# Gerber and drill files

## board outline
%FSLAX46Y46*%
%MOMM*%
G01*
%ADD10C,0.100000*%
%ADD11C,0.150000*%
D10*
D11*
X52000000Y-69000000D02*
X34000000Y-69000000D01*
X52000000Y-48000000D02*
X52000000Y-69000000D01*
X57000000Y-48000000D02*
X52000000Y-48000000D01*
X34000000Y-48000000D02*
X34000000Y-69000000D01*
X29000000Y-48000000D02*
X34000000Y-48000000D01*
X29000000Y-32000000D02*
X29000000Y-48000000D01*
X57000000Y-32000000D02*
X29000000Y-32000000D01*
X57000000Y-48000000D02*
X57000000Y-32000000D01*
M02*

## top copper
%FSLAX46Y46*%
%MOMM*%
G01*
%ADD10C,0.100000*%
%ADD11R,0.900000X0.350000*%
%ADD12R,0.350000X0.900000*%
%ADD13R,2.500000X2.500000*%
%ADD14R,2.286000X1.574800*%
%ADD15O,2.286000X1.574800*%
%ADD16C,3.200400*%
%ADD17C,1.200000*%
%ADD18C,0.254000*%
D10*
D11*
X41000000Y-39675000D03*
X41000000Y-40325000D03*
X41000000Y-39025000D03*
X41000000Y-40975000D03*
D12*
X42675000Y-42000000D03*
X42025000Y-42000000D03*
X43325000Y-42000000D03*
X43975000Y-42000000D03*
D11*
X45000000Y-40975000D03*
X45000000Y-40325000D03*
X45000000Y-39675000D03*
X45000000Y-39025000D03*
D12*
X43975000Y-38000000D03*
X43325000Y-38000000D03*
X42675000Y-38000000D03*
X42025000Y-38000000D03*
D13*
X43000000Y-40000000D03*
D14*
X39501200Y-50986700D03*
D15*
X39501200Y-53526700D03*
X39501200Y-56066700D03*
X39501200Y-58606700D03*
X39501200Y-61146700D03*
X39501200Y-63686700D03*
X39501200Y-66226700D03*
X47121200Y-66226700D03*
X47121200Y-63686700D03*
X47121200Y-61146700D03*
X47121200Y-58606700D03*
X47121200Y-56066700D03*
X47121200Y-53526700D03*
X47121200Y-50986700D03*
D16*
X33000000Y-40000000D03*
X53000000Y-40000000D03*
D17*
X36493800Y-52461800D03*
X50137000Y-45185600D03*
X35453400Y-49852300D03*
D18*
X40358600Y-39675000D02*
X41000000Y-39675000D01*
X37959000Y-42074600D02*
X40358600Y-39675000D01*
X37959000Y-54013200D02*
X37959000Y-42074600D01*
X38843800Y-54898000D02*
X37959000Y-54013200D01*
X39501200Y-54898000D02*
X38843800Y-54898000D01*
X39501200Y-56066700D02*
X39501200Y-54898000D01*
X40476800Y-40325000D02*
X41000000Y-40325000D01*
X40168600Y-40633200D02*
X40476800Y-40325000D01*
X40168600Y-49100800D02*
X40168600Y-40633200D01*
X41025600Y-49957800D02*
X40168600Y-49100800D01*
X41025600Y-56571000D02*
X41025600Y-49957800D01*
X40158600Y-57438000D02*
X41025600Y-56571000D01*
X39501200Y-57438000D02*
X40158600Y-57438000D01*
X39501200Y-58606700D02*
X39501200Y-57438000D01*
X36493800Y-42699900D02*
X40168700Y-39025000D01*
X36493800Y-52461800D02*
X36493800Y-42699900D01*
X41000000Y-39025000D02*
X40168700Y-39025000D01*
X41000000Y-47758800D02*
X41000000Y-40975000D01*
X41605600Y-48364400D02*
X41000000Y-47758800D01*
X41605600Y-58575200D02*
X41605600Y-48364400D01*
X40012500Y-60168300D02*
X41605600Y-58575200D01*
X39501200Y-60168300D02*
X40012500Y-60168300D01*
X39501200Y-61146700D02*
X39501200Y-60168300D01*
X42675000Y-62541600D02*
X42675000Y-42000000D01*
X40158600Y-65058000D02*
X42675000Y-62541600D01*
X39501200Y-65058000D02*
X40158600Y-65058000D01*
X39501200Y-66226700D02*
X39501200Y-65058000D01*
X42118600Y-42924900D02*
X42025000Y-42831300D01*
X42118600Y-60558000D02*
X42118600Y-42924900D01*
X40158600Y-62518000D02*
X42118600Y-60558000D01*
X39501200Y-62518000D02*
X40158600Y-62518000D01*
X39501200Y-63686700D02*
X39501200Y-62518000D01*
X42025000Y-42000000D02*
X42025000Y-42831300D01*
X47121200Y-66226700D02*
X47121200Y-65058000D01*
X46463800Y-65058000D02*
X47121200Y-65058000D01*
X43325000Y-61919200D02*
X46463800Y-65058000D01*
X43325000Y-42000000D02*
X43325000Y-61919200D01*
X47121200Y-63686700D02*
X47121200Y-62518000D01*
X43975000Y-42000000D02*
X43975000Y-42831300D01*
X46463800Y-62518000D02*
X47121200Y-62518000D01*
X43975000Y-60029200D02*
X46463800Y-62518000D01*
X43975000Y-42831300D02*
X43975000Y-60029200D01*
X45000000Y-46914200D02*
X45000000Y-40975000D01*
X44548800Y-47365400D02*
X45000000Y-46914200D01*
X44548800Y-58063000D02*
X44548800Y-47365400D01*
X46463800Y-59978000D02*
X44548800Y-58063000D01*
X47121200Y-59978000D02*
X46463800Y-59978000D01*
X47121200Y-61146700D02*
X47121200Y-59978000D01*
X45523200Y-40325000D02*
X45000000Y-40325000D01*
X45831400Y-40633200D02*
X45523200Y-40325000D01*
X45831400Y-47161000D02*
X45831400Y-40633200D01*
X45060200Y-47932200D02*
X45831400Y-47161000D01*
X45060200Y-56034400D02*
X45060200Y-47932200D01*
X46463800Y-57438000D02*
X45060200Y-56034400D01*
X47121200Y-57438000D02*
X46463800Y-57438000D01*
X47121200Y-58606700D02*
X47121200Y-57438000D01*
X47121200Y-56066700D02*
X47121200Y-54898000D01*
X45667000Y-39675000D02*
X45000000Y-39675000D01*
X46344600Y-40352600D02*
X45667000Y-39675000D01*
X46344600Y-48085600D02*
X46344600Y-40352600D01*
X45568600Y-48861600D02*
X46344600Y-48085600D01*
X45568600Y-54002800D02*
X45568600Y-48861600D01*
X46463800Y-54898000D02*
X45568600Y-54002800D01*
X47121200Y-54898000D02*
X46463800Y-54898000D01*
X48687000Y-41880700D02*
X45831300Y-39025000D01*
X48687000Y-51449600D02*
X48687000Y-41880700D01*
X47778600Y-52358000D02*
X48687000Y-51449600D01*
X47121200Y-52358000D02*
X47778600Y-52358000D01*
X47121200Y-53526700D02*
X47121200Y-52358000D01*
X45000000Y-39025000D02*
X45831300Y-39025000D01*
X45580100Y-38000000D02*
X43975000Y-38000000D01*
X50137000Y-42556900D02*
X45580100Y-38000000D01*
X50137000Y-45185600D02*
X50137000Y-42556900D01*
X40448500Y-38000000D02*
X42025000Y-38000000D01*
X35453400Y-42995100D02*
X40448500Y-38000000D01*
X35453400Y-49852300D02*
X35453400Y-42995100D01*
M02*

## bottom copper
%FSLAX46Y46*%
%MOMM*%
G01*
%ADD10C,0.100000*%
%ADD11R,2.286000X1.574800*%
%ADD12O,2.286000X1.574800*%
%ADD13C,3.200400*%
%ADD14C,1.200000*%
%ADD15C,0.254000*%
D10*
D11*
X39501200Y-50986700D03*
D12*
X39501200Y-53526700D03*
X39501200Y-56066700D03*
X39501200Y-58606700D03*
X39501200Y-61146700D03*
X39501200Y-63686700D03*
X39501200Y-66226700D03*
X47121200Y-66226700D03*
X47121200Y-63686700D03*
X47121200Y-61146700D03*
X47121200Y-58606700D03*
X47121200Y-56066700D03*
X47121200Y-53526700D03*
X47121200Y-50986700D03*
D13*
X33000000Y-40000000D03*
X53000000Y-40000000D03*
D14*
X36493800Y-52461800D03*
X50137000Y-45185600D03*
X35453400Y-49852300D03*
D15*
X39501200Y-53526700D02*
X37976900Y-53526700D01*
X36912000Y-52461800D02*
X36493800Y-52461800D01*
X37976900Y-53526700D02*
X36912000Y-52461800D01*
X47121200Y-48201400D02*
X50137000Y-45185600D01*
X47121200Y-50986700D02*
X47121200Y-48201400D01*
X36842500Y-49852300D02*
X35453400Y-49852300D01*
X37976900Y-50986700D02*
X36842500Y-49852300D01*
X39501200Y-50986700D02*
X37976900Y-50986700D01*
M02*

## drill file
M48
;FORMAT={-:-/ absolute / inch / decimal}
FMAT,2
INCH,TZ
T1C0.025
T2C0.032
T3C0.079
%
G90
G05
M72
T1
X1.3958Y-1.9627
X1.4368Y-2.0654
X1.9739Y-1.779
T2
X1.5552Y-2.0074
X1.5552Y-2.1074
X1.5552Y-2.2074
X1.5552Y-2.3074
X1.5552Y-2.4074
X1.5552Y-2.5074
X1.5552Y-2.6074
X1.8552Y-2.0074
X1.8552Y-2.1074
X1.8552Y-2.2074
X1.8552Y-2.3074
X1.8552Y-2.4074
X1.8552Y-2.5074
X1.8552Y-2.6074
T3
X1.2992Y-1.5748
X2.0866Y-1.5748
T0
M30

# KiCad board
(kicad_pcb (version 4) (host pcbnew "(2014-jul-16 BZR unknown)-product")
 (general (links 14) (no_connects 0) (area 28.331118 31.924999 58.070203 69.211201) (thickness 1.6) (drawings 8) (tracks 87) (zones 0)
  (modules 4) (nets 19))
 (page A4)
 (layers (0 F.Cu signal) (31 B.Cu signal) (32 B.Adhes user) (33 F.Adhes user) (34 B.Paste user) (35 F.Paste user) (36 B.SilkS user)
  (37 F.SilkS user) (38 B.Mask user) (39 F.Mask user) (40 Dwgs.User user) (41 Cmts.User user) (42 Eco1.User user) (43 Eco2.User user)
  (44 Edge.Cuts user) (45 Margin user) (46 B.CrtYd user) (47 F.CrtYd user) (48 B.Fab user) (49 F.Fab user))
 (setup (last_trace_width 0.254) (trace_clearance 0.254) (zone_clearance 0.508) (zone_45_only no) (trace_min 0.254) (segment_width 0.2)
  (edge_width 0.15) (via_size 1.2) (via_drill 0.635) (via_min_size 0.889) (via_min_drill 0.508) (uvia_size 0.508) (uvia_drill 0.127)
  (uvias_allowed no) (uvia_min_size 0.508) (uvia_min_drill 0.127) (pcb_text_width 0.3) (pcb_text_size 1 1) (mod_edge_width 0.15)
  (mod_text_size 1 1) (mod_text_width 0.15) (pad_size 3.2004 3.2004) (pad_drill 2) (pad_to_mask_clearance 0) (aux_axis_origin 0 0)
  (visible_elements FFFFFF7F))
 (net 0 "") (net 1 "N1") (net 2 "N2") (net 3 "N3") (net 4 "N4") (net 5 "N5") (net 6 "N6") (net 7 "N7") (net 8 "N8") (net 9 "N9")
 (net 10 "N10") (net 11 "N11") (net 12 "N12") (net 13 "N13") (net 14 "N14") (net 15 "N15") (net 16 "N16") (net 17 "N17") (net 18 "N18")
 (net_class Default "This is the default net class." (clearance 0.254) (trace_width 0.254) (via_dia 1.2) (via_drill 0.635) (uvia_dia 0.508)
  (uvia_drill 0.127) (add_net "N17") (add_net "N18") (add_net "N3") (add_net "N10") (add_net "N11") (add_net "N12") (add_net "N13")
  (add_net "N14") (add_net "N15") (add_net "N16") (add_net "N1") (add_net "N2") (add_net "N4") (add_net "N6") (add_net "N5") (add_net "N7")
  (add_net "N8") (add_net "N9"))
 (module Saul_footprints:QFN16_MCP (layer F.Cu) (at 43 40)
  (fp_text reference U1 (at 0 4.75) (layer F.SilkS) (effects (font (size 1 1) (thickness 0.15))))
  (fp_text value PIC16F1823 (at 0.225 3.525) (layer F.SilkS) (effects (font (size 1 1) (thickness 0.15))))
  (pad 2 smd rect (at -2 -0.325) (size 0.9 0.35) (layers F.Cu F.Paste F.Mask) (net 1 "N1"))
  (pad 3 smd rect (at -2 0.325) (size 0.9 0.35) (layers F.Cu F.Paste F.Mask) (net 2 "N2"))
  (pad 1 smd rect (at -2 -0.975) (size 0.9 0.35) (layers F.Cu F.Paste F.Mask) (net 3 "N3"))
  (pad 4 smd rect (at -2 0.975) (size 0.9 0.35) (layers F.Cu F.Paste F.Mask) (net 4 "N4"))
  (pad 6 smd rect (at -0.325 2 90) (size 0.9 0.35) (layers F.Cu F.Paste F.Mask) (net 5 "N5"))
  (pad 5 smd rect (at -0.975 2 90) (size 0.9 0.35) (layers F.Cu F.Paste F.Mask) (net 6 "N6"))
  (pad 7 smd rect (at 0.325 2 90) (size 0.9 0.35) (layers F.Cu F.Paste F.Mask) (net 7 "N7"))
  (pad 8 smd rect (at 0.975 2 90) (size 0.9 0.35) (layers F.Cu F.Paste F.Mask) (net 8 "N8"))
  (pad 9 smd rect (at 2 0.975) (size 0.9 0.35) (layers F.Cu F.Paste F.Mask) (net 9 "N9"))
  (pad 10 smd rect (at 2 0.325) (size 0.9 0.35) (layers F.Cu F.Paste F.Mask) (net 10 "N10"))
  (pad 11 smd rect (at 2 -0.325) (size 0.9 0.35) (layers F.Cu F.Paste F.Mask) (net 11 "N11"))
  (pad 12 smd rect (at 2 -0.975) (size 0.9 0.35) (layers F.Cu F.Paste F.Mask) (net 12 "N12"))
  (pad 13 smd rect (at 0.975 -2 90) (size 0.9 0.35) (layers F.Cu F.Paste F.Mask) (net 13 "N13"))
  (pad 14 smd rect (at 0.325 -2 90) (size 0.9 0.35) (layers F.Cu F.Paste F.Mask) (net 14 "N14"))
  (pad 15 smd rect (at -0.325 -2 90) (size 0.9 0.35) (layers F.Cu F.Paste F.Mask) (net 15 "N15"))
  (pad 16 smd rect (at -0.975 -2 90) (size 0.9 0.35) (layers F.Cu F.Paste F.Mask) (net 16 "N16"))
  (pad "" smd rect (at 0 0 90) (size 2.5 2.5) (layers F.Cu F.Paste F.Mask)))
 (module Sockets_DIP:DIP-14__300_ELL (layer F.Cu) (at 43.3112 58.6067 270)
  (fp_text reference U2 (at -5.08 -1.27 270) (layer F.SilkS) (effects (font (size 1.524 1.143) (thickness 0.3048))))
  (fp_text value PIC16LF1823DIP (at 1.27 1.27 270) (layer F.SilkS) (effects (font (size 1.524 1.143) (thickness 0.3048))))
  (pad 1 thru_hole rect (at -7.62 3.81 270) (size 1.5748 2.286) (drill 0.8128) (layers *.Cu *.Mask F.SilkS) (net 16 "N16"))
  (pad 2 thru_hole oval (at -5.08 3.81 270) (size 1.5748 2.286) (drill 0.8128) (layers *.Cu *.Mask F.SilkS) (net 3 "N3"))
  (pad 3 thru_hole oval (at -2.54 3.81 270) (size 1.5748 2.286) (drill 0.8128) (layers *.Cu *.Mask F.SilkS) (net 1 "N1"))
  (pad 4 thru_hole oval (at 0 3.81 270) (size 1.5748 2.286) (drill 0.8128) (layers *.Cu *.Mask F.SilkS) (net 2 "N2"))
  (pad 5 thru_hole oval (at 2.54 3.81 270) (size 1.5748 2.286) (drill 0.8128) (layers *.Cu *.Mask F.SilkS) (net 4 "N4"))
  (pad 6 thru_hole oval (at 5.08 3.81 270) (size 1.5748 2.286) (drill 0.8128) (layers *.Cu *.Mask F.SilkS) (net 6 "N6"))
  (pad 7 thru_hole oval (at 7.62 3.81 270) (size 1.5748 2.286) (drill 0.8128) (layers *.Cu *.Mask F.SilkS) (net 5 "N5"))
  (pad 8 thru_hole oval (at 7.62 -3.81 270) (size 1.5748 2.286) (drill 0.8128) (layers *.Cu *.Mask F.SilkS) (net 7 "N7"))
  (pad 9 thru_hole oval (at 5.08 -3.81 270) (size 1.5748 2.286) (drill 0.8128) (layers *.Cu *.Mask F.SilkS) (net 8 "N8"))
  (pad 10 thru_hole oval (at 2.54 -3.81 270) (size 1.5748 2.286) (drill 0.8128) (layers *.Cu *.Mask F.SilkS) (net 9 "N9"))
  (pad 11 thru_hole oval (at 0 -3.81 270) (size 1.5748 2.286) (drill 0.8128) (layers *.Cu *.Mask F.SilkS) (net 10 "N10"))
  (pad 12 thru_hole oval (at -2.54 -3.81 270) (size 1.5748 2.286) (drill 0.8128) (layers *.Cu *.Mask F.SilkS) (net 11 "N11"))
  (pad 13 thru_hole oval (at -5.08 -3.81 270) (size 1.5748 2.286) (drill 0.8128) (layers *.Cu *.Mask F.SilkS) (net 12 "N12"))
  (pad 14 thru_hole oval (at -7.62 -3.81 270) (size 1.5748 2.286) (drill 0.8128) (layers *.Cu *.Mask F.SilkS) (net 13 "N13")))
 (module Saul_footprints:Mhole (layer F.Cu) (at 33 40)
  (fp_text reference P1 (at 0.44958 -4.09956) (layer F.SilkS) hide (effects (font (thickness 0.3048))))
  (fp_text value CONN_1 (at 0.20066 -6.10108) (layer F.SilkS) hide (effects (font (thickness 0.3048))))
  (pad 1 thru_hole circle (at 0 0) (size 3.2004 3.2004) (drill 2) (layers *.Cu *.Mask F.SilkS) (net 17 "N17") (clearance 1.00076)))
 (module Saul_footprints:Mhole (layer F.Cu) (at 53 40)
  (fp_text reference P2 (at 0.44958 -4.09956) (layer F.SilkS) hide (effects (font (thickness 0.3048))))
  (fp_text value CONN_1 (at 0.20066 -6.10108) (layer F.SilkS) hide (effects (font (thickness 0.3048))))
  (pad 1 thru_hole circle (at 0 0) (size 3.2004 3.2004) (drill 2) (layers *.Cu *.Mask F.SilkS) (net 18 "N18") (clearance 1.00076)))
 (gr_line (start 52 69) (end 34 69) (angle 90) (layer Edge.Cuts) (width 0.15))
 (gr_line (start 52 48) (end 52 69) (angle 90) (layer Edge.Cuts) (width 0.15))
 (gr_line (start 57 48) (end 52 48) (angle 90) (layer Edge.Cuts) (width 0.15))
 (gr_line (start 34 48) (end 34 69) (angle 90) (layer Edge.Cuts) (width 0.15))
 (gr_line (start 29 48) (end 34 48) (angle 90) (layer Edge.Cuts) (width 0.15))
 (gr_line (start 29 32) (end 29 48) (angle 90) (layer Edge.Cuts) (width 0.15))
 (gr_line (start 57 32) (end 29 32) (angle 90) (layer Edge.Cuts) (width 0.15))
 (gr_line (start 57 48) (end 57 32) (angle 90) (layer Edge.Cuts) (width 0.15))
 (segment (start 40.3586 39.675) (end 41 39.675) (width 0.254) (layer F.Cu) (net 1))
 (segment (start 37.959 42.0746) (end 40.3586 39.675) (width 0.254) (layer F.Cu) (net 1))
 (segment (start 37.959 54.0132) (end 37.959 42.0746) (width 0.254) (layer F.Cu) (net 1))
 (segment (start 38.8438 54.898) (end 37.959 54.0132) (width 0.254) (layer F.Cu) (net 1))
 (segment (start 39.5012 54.898) (end 38.8438 54.898) (width 0.254) (layer F.Cu) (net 1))
 (segment (start 39.5012 56.0667) (end 39.5012 54.898) (width 0.254) (layer F.Cu) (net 1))
 (segment (start 40.4768 40.325) (end 41 40.325) (width 0.254) (layer F.Cu) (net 2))
 (segment (start 40.1686 40.6332) (end 40.4768 40.325) (width 0.254) (layer F.Cu) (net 2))
 (segment (start 40.1686 49.1008) (end 40.1686 40.6332) (width 0.254) (layer F.Cu) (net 2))
 (segment (start 41.0256 49.9578) (end 40.1686 49.1008) (width 0.254) (layer F.Cu) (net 2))
 (segment (start 41.0256 56.571) (end 41.0256 49.9578) (width 0.254) (layer F.Cu) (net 2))
 (segment (start 40.1586 57.438) (end 41.0256 56.571) (width 0.254) (layer F.Cu) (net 2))
 (segment (start 39.5012 57.438) (end 40.1586 57.438) (width 0.254) (layer F.Cu) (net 2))
 (segment (start 39.5012 58.6067) (end 39.5012 57.438) (width 0.254) (layer F.Cu) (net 2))
 (via (at 36.4938 52.4618) (size 1.2) (layers F.Cu B.Cu) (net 3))
 (segment (start 39.5012 53.5267) (end 37.9769 53.5267) (width 0.254) (layer B.Cu) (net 3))
 (segment (start 36.912 52.4618) (end 36.4938 52.4618) (width 0.254) (layer B.Cu) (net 3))
 (segment (start 37.9769 53.5267) (end 36.912 52.4618) (width 0.254) (layer B.Cu) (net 3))
 (segment (start 36.4938 42.6999) (end 40.1687 39.025) (width 0.254) (layer F.Cu) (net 3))
 (segment (start 36.4938 52.4618) (end 36.4938 42.6999) (width 0.254) (layer F.Cu) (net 3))
 (segment (start 41 39.025) (end 40.1687 39.025) (width 0.254) (layer F.Cu) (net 3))
 (segment (start 41 47.7588) (end 41 40.975) (width 0.254) (layer F.Cu) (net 4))
 (segment (start 41.6056 48.3644) (end 41 47.7588) (width 0.254) (layer F.Cu) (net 4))
 (segment (start 41.6056 58.5752) (end 41.6056 48.3644) (width 0.254) (layer F.Cu) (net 4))
 (segment (start 40.0125 60.1683) (end 41.6056 58.5752) (width 0.254) (layer F.Cu) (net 4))
 (segment (start 39.5012 60.1683) (end 40.0125 60.1683) (width 0.254) (layer F.Cu) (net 4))
 (segment (start 39.5012 61.1467) (end 39.5012 60.1683) (width 0.254) (layer F.Cu) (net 4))
 (segment (start 42.675 62.5416) (end 42.675 42) (width 0.254) (layer F.Cu) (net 5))
 (segment (start 40.1586 65.058) (end 42.675 62.5416) (width 0.254) (layer F.Cu) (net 5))
 (segment (start 39.5012 65.058) (end 40.1586 65.058) (width 0.254) (layer F.Cu) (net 5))
 (segment (start 39.5012 66.2267) (end 39.5012 65.058) (width 0.254) (layer F.Cu) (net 5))
 (segment (start 42.1186 42.9249) (end 42.025 42.8313) (width 0.254) (layer F.Cu) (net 6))
 (segment (start 42.1186 60.558) (end 42.1186 42.9249) (width 0.254) (layer F.Cu) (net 6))
 (segment (start 40.1586 62.518) (end 42.1186 60.558) (width 0.254) (layer F.Cu) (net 6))
 (segment (start 39.5012 62.518) (end 40.1586 62.518) (width 0.254) (layer F.Cu) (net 6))
 (segment (start 39.5012 63.6867) (end 39.5012 62.518) (width 0.254) (layer F.Cu) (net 6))
 (segment (start 42.025 42) (end 42.025 42.8313) (width 0.254) (layer F.Cu) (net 6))
 (segment (start 47.1212 66.2267) (end 47.1212 65.058) (width 0.254) (layer F.Cu) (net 7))
 (segment (start 46.4638 65.058) (end 47.1212 65.058) (width 0.254) (layer F.Cu) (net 7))
 (segment (start 43.325 61.9192) (end 46.4638 65.058) (width 0.254) (layer F.Cu) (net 7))
 (segment (start 43.325 42) (end 43.325 61.9192) (width 0.254) (layer F.Cu) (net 7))
 (segment (start 47.1212 63.6867) (end 47.1212 62.518) (width 0.254) (layer F.Cu) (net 8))
 (segment (start 43.975 42) (end 43.975 42.8313) (width 0.254) (layer F.Cu) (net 8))
 (segment (start 46.4638 62.518) (end 47.1212 62.518) (width 0.254) (layer F.Cu) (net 8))
 (segment (start 43.975 60.0292) (end 46.4638 62.518) (width 0.254) (layer F.Cu) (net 8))
 (segment (start 43.975 42.8313) (end 43.975 60.0292) (width 0.254) (layer F.Cu) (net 8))
 (segment (start 45 46.9142) (end 45 40.975) (width 0.254) (layer F.Cu) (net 9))
 (segment (start 44.5488 47.3654) (end 45 46.9142) (width 0.254) (layer F.Cu) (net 9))
 (segment (start 44.5488 58.063) (end 44.5488 47.3654) (width 0.254) (layer F.Cu) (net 9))
 (segment (start 46.4638 59.978) (end 44.5488 58.063) (width 0.254) (layer F.Cu) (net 9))
 (segment (start 47.1212 59.978) (end 46.4638 59.978) (width 0.254) (layer F.Cu) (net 9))
 (segment (start 47.1212 61.1467) (end 47.1212 59.978) (width 0.254) (layer F.Cu) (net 9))
 (segment (start 45.5232 40.325) (end 45 40.325) (width 0.254) (layer F.Cu) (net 10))
 (segment (start 45.8314 40.6332) (end 45.5232 40.325) (width 0.254) (layer F.Cu) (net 10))
 (segment (start 45.8314 47.161) (end 45.8314 40.6332) (width 0.254) (layer F.Cu) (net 10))
 (segment (start 45.0602 47.9322) (end 45.8314 47.161) (width 0.254) (layer F.Cu) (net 10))
 (segment (start 45.0602 56.0344) (end 45.0602 47.9322) (width 0.254) (layer F.Cu) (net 10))
 (segment (start 46.4638 57.438) (end 45.0602 56.0344) (width 0.254) (layer F.Cu) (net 10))
 (segment (start 47.1212 57.438) (end 46.4638 57.438) (width 0.254) (layer F.Cu) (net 10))
 (segment (start 47.1212 58.6067) (end 47.1212 57.438) (width 0.254) (layer F.Cu) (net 10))
 (segment (start 47.1212 56.0667) (end 47.1212 54.898) (width 0.254) (layer F.Cu) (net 11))
 (segment (start 45.667 39.675) (end 45 39.675) (width 0.254) (layer F.Cu) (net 11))
 (segment (start 46.3446 40.3526) (end 45.667 39.675) (width 0.254) (layer F.Cu) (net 11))
 (segment (start 46.3446 48.0856) (end 46.3446 40.3526) (width 0.254) (layer F.Cu) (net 11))
 (segment (start 45.5686 48.8616) (end 46.3446 48.0856) (width 0.254) (layer F.Cu) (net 11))
 (segment (start 45.5686 54.0028) (end 45.5686 48.8616) (width 0.254) (layer F.Cu) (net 11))
 (segment (start 46.4638 54.898) (end 45.5686 54.0028) (width 0.254) (layer F.Cu) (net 11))
 (segment (start 47.1212 54.898) (end 46.4638 54.898) (width 0.254) (layer F.Cu) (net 11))
 (segment (start 48.687 41.8807) (end 45.8313 39.025) (width 0.254) (layer F.Cu) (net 12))
 (segment (start 48.687 51.4496) (end 48.687 41.8807) (width 0.254) (layer F.Cu) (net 12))
 (segment (start 47.7786 52.358) (end 48.687 51.4496) (width 0.254) (layer F.Cu) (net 12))
 (segment (start 47.1212 52.358) (end 47.7786 52.358) (width 0.254) (layer F.Cu) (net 12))
 (segment (start 47.1212 53.5267) (end 47.1212 52.358) (width 0.254) (layer F.Cu) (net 12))
 (segment (start 45 39.025) (end 45.8313 39.025) (width 0.254) (layer F.Cu) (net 12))
 (via (at 50.137 45.1856) (size 1.2) (layers F.Cu B.Cu) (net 13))
 (segment (start 47.1212 48.2014) (end 50.137 45.1856) (width 0.254) (layer B.Cu) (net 13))
 (segment (start 47.1212 50.9867) (end 47.1212 48.2014) (width 0.254) (layer B.Cu) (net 13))
 (segment (start 45.5801 38) (end 43.975 38) (width 0.254) (layer F.Cu) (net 13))
 (segment (start 50.137 42.5569) (end 45.5801 38) (width 0.254) (layer F.Cu) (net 13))
 (segment (start 50.137 45.1856) (end 50.137 42.5569) (width 0.254) (layer F.Cu) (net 13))
 (via (at 35.4534 49.8523) (size 1.2) (layers F.Cu B.Cu) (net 16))
 (segment (start 36.8425 49.8523) (end 35.4534 49.8523) (width 0.254) (layer B.Cu) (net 16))
 (segment (start 37.9769 50.9867) (end 36.8425 49.8523) (width 0.254) (layer B.Cu) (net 16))
 (segment (start 40.4485 38) (end 42.025 38) (width 0.254) (layer F.Cu) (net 16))
 (segment (start 35.4534 42.9951) (end 40.4485 38) (width 0.254) (layer F.Cu) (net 16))
 (segment (start 35.4534 49.8523) (end 35.4534 42.9951) (width 0.254) (layer F.Cu) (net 16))
 (segment (start 39.5012 50.9867) (end 37.9769 50.9867) (width 0.254) (layer B.Cu) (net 16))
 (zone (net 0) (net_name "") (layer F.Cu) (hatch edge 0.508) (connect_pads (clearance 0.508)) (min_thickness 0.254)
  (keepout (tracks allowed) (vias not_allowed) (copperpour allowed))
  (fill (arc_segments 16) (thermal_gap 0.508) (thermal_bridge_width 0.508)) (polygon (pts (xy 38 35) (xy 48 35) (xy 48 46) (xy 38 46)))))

